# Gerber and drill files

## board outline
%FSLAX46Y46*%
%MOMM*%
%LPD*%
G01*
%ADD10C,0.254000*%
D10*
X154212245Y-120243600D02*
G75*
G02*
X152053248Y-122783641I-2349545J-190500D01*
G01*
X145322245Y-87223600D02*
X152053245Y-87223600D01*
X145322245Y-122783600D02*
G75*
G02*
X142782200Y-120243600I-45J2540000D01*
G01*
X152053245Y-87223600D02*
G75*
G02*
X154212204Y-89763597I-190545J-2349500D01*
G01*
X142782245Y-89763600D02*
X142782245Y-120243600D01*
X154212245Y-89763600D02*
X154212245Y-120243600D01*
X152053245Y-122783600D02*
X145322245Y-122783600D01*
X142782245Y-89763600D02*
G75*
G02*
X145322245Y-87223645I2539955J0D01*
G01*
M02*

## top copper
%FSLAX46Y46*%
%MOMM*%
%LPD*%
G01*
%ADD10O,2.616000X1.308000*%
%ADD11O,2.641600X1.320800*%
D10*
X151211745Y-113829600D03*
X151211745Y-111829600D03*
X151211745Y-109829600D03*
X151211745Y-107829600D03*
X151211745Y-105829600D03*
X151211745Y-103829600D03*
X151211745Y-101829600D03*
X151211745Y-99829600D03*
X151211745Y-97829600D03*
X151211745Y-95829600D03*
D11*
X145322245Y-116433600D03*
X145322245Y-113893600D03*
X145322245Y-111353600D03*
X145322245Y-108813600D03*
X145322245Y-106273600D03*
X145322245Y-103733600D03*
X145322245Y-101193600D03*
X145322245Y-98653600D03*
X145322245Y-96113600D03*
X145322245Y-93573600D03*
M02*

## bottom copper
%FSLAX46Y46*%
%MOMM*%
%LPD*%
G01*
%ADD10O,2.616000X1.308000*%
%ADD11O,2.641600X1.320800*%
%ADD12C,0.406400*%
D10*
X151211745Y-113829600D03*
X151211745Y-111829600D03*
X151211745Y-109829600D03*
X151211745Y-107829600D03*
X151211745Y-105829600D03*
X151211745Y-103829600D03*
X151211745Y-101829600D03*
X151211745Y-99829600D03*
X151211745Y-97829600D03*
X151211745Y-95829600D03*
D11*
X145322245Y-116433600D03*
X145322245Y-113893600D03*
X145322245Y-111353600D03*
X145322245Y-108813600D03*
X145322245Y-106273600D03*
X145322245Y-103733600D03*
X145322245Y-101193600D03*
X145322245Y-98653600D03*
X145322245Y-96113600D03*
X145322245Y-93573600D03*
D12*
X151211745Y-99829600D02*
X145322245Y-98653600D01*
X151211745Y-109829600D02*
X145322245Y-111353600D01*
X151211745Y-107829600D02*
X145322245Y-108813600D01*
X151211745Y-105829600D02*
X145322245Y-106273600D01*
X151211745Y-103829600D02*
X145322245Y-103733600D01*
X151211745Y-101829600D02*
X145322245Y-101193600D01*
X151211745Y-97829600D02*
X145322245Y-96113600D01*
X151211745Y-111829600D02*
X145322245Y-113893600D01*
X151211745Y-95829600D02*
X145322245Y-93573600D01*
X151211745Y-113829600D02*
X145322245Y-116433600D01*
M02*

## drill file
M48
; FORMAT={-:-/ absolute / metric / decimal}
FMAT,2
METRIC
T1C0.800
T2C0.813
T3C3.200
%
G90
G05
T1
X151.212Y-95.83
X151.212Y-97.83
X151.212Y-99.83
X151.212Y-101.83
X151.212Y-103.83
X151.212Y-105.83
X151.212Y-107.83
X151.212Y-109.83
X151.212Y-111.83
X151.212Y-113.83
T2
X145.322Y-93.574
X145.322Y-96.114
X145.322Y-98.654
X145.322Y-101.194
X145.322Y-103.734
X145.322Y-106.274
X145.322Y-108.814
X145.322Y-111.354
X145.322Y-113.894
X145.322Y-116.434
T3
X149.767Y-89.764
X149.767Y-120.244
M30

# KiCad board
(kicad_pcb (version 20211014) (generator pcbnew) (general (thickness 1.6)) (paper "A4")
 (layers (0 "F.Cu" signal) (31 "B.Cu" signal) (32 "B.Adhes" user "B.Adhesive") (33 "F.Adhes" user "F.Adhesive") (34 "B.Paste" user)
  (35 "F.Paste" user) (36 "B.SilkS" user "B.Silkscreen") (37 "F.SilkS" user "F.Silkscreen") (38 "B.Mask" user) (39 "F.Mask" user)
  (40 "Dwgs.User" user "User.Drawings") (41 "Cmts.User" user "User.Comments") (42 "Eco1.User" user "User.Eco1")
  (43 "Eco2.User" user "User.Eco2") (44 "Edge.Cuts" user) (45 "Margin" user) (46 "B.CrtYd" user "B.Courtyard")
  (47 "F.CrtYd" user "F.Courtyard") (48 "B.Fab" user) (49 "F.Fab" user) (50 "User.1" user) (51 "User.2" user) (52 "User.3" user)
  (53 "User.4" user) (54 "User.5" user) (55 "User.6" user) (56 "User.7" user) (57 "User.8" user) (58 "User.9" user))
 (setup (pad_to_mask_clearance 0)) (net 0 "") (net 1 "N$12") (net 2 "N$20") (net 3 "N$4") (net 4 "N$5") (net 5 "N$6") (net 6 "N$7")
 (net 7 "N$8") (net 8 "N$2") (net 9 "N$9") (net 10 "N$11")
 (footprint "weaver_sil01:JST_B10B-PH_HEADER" (layer "F.Cu") (at 151.164245 109.8296 -90)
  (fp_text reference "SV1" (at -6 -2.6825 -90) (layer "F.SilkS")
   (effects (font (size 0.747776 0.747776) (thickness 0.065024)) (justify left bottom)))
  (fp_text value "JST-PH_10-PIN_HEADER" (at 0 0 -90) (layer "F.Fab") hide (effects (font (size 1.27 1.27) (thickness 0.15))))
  (pad "P1" thru_hole oval (at 4 -0.0475) (size 2.616 1.308) (drill 0.8) (layers *.Cu *.Mask) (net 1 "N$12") (solder_mask_margin 0.1016))
  (pad "P2" thru_hole oval (at 2 -0.0475) (size 2.616 1.308) (drill 0.8) (layers *.Cu *.Mask) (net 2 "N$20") (solder_mask_margin 0.1016))
  (pad "P3" thru_hole oval (at 0 -0.0475) (size 2.616 1.308) (drill 0.8) (layers *.Cu *.Mask) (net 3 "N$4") (solder_mask_margin 0.1016))
  (pad "P4" thru_hole oval (at -2 -0.0475) (size 2.616 1.308) (drill 0.8) (layers *.Cu *.Mask) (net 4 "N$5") (solder_mask_margin 0.1016))
  (pad "P5" thru_hole oval (at -4 -0.0475) (size 2.616 1.308) (drill 0.8) (layers *.Cu *.Mask) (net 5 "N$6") (solder_mask_margin 0.1016))
  (pad "P6" thru_hole oval (at -6 -0.0475) (size 2.616 1.308) (drill 0.8) (layers *.Cu *.Mask) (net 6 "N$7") (solder_mask_margin 0.1016))
  (pad "P7" thru_hole oval (at -8 -0.0475) (size 2.616 1.308) (drill 0.8) (layers *.Cu *.Mask) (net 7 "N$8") (solder_mask_margin 0.1016))
  (pad "P8" thru_hole oval (at -10 -0.0475) (size 2.616 1.308) (drill 0.8) (layers *.Cu *.Mask) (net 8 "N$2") (solder_mask_margin 0.1016))
  (pad "P9" thru_hole oval (at -12 -0.0475) (size 2.616 1.308) (drill 0.8) (layers *.Cu *.Mask) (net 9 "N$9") (solder_mask_margin 0.1016))
  (pad "P10" thru_hole oval (at -14 -0.0475) (size 2.616 1.308) (drill 0.8) (layers *.Cu *.Mask) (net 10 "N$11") (solder_mask_margin 0.1016)))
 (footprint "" (layer "F.Cu") (at 149.767245 120.2436)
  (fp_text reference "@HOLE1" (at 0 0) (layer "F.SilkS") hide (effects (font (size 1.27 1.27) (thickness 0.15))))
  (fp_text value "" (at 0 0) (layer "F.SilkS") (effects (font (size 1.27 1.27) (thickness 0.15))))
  (pad "" np_thru_hole circle (at 0 0) (size 3.2 3.2) (drill 3.2) (layers *.Cu *.Mask)))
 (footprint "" (layer "F.Cu") (at 149.767245 89.7636)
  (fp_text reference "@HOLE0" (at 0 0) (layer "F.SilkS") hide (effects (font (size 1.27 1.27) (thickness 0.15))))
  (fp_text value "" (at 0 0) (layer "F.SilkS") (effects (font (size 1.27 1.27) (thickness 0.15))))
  (pad "" np_thru_hole circle (at 0 0) (size 3.2 3.2) (drill 3.2) (layers *.Cu *.Mask)))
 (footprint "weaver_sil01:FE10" (layer "F.Cu") (at 145.322245 105.0036 90)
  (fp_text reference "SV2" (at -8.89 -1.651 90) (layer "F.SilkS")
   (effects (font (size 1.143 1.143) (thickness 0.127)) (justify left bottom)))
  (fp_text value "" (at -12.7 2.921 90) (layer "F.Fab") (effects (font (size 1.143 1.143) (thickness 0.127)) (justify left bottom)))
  (pad "1" thru_hole oval (at -11.43 0 180) (size 2.6416 1.3208) (drill 0.8128) (layers *.Cu *.Mask) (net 1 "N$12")
   (solder_mask_margin 0.1016))
  (pad "2" thru_hole oval (at -8.89 0 180) (size 2.6416 1.3208) (drill 0.8128) (layers *.Cu *.Mask) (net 2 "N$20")
   (solder_mask_margin 0.1016))
  (pad "3" thru_hole oval (at -6.35 0 180) (size 2.6416 1.3208) (drill 0.8128) (layers *.Cu *.Mask) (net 3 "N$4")
   (solder_mask_margin 0.1016))
  (pad "4" thru_hole oval (at -3.81 0 180) (size 2.6416 1.3208) (drill 0.8128) (layers *.Cu *.Mask) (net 4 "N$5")
   (solder_mask_margin 0.1016))
  (pad "5" thru_hole oval (at -1.27 0 180) (size 2.6416 1.3208) (drill 0.8128) (layers *.Cu *.Mask) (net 5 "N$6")
   (solder_mask_margin 0.1016))
  (pad "6" thru_hole oval (at 1.27 0 180) (size 2.6416 1.3208) (drill 0.8128) (layers *.Cu *.Mask) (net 6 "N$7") (solder_mask_margin 0.1016))
  (pad "7" thru_hole oval (at 3.81 0 180) (size 2.6416 1.3208) (drill 0.8128) (layers *.Cu *.Mask) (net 7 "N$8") (solder_mask_margin 0.1016))
  (pad "8" thru_hole oval (at 6.35 0 180) (size 2.6416 1.3208) (drill 0.8128) (layers *.Cu *.Mask) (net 8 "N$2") (solder_mask_margin 0.1016))
  (pad "9" thru_hole oval (at 8.89 0 180) (size 2.6416 1.3208) (drill 0.8128) (layers *.Cu *.Mask) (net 9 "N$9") (solder_mask_margin 0.1016))
  (pad "10" thru_hole oval (at 11.43 0 180) (size 2.6416 1.3208) (drill 0.8128) (layers *.Cu *.Mask) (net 10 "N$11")
   (solder_mask_margin 0.1016)))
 (gr_arc (start 154.212245 120.2436) (mid 153.658796 121.960744) (end 152.053245 122.7836) (layer "Edge.Cuts") (width 0.254))
 (gr_line (start 145.322245 87.2236) (end 152.053245 87.2236) (layer "Edge.Cuts") (width 0.254))
 (gr_arc (start 145.322245 122.7836) (mid 143.526194 122.039651) (end 142.782245 120.2436) (layer "Edge.Cuts") (width 0.254))
 (gr_arc (start 152.053245 87.2236) (mid 153.658796 88.046456) (end 154.212245 89.7636) (layer "Edge.Cuts") (width 0.254))
 (gr_line (start 142.782245 89.7636) (end 142.782245 120.2436) (layer "Edge.Cuts") (width 0.254))
 (gr_line (start 154.212245 89.7636) (end 154.212245 120.2436) (layer "Edge.Cuts") (width 0.254))
 (gr_line (start 152.053245 122.7836) (end 145.322245 122.7836) (layer "Edge.Cuts") (width 0.254))
 (gr_arc (start 142.782245 89.7636) (mid 143.526194 87.967549) (end 145.322245 87.2236) (layer "Edge.Cuts") (width 0.254))
 (segment (start 151.211745 99.8296) (end 145.322245 98.6536) (width 0.4064) (layer "B.Cu") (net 8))
 (segment (start 151.211745 109.8296) (end 145.322245 111.3536) (width 0.4064) (layer "B.Cu") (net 3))
 (segment (start 151.211745 107.8296) (end 145.322245 108.8136) (width 0.4064) (layer "B.Cu") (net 4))
 (segment (start 151.211745 105.8296) (end 145.322245 106.2736) (width 0.4064) (layer "B.Cu") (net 5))
 (segment (start 151.211745 103.8296) (end 145.322245 103.7336) (width 0.4064) (layer "B.Cu") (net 6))
 (segment (start 151.211745 101.8296) (end 145.322245 101.1936) (width 0.4064) (layer "B.Cu") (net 7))
 (segment (start 151.211745 97.8296) (end 145.322245 96.1136) (width 0.4064) (layer "B.Cu") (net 9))
 (segment (start 151.211745 111.8296) (end 145.322245 113.8936) (width 0.4064) (layer "B.Cu") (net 2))
 (segment (start 151.211745 95.8296) (end 145.322245 93.5736) (width 0.4064) (layer "B.Cu") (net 10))
 (segment (start 151.211745 113.8296) (end 145.322245 116.4336) (width 0.4064) (layer "B.Cu") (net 1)))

